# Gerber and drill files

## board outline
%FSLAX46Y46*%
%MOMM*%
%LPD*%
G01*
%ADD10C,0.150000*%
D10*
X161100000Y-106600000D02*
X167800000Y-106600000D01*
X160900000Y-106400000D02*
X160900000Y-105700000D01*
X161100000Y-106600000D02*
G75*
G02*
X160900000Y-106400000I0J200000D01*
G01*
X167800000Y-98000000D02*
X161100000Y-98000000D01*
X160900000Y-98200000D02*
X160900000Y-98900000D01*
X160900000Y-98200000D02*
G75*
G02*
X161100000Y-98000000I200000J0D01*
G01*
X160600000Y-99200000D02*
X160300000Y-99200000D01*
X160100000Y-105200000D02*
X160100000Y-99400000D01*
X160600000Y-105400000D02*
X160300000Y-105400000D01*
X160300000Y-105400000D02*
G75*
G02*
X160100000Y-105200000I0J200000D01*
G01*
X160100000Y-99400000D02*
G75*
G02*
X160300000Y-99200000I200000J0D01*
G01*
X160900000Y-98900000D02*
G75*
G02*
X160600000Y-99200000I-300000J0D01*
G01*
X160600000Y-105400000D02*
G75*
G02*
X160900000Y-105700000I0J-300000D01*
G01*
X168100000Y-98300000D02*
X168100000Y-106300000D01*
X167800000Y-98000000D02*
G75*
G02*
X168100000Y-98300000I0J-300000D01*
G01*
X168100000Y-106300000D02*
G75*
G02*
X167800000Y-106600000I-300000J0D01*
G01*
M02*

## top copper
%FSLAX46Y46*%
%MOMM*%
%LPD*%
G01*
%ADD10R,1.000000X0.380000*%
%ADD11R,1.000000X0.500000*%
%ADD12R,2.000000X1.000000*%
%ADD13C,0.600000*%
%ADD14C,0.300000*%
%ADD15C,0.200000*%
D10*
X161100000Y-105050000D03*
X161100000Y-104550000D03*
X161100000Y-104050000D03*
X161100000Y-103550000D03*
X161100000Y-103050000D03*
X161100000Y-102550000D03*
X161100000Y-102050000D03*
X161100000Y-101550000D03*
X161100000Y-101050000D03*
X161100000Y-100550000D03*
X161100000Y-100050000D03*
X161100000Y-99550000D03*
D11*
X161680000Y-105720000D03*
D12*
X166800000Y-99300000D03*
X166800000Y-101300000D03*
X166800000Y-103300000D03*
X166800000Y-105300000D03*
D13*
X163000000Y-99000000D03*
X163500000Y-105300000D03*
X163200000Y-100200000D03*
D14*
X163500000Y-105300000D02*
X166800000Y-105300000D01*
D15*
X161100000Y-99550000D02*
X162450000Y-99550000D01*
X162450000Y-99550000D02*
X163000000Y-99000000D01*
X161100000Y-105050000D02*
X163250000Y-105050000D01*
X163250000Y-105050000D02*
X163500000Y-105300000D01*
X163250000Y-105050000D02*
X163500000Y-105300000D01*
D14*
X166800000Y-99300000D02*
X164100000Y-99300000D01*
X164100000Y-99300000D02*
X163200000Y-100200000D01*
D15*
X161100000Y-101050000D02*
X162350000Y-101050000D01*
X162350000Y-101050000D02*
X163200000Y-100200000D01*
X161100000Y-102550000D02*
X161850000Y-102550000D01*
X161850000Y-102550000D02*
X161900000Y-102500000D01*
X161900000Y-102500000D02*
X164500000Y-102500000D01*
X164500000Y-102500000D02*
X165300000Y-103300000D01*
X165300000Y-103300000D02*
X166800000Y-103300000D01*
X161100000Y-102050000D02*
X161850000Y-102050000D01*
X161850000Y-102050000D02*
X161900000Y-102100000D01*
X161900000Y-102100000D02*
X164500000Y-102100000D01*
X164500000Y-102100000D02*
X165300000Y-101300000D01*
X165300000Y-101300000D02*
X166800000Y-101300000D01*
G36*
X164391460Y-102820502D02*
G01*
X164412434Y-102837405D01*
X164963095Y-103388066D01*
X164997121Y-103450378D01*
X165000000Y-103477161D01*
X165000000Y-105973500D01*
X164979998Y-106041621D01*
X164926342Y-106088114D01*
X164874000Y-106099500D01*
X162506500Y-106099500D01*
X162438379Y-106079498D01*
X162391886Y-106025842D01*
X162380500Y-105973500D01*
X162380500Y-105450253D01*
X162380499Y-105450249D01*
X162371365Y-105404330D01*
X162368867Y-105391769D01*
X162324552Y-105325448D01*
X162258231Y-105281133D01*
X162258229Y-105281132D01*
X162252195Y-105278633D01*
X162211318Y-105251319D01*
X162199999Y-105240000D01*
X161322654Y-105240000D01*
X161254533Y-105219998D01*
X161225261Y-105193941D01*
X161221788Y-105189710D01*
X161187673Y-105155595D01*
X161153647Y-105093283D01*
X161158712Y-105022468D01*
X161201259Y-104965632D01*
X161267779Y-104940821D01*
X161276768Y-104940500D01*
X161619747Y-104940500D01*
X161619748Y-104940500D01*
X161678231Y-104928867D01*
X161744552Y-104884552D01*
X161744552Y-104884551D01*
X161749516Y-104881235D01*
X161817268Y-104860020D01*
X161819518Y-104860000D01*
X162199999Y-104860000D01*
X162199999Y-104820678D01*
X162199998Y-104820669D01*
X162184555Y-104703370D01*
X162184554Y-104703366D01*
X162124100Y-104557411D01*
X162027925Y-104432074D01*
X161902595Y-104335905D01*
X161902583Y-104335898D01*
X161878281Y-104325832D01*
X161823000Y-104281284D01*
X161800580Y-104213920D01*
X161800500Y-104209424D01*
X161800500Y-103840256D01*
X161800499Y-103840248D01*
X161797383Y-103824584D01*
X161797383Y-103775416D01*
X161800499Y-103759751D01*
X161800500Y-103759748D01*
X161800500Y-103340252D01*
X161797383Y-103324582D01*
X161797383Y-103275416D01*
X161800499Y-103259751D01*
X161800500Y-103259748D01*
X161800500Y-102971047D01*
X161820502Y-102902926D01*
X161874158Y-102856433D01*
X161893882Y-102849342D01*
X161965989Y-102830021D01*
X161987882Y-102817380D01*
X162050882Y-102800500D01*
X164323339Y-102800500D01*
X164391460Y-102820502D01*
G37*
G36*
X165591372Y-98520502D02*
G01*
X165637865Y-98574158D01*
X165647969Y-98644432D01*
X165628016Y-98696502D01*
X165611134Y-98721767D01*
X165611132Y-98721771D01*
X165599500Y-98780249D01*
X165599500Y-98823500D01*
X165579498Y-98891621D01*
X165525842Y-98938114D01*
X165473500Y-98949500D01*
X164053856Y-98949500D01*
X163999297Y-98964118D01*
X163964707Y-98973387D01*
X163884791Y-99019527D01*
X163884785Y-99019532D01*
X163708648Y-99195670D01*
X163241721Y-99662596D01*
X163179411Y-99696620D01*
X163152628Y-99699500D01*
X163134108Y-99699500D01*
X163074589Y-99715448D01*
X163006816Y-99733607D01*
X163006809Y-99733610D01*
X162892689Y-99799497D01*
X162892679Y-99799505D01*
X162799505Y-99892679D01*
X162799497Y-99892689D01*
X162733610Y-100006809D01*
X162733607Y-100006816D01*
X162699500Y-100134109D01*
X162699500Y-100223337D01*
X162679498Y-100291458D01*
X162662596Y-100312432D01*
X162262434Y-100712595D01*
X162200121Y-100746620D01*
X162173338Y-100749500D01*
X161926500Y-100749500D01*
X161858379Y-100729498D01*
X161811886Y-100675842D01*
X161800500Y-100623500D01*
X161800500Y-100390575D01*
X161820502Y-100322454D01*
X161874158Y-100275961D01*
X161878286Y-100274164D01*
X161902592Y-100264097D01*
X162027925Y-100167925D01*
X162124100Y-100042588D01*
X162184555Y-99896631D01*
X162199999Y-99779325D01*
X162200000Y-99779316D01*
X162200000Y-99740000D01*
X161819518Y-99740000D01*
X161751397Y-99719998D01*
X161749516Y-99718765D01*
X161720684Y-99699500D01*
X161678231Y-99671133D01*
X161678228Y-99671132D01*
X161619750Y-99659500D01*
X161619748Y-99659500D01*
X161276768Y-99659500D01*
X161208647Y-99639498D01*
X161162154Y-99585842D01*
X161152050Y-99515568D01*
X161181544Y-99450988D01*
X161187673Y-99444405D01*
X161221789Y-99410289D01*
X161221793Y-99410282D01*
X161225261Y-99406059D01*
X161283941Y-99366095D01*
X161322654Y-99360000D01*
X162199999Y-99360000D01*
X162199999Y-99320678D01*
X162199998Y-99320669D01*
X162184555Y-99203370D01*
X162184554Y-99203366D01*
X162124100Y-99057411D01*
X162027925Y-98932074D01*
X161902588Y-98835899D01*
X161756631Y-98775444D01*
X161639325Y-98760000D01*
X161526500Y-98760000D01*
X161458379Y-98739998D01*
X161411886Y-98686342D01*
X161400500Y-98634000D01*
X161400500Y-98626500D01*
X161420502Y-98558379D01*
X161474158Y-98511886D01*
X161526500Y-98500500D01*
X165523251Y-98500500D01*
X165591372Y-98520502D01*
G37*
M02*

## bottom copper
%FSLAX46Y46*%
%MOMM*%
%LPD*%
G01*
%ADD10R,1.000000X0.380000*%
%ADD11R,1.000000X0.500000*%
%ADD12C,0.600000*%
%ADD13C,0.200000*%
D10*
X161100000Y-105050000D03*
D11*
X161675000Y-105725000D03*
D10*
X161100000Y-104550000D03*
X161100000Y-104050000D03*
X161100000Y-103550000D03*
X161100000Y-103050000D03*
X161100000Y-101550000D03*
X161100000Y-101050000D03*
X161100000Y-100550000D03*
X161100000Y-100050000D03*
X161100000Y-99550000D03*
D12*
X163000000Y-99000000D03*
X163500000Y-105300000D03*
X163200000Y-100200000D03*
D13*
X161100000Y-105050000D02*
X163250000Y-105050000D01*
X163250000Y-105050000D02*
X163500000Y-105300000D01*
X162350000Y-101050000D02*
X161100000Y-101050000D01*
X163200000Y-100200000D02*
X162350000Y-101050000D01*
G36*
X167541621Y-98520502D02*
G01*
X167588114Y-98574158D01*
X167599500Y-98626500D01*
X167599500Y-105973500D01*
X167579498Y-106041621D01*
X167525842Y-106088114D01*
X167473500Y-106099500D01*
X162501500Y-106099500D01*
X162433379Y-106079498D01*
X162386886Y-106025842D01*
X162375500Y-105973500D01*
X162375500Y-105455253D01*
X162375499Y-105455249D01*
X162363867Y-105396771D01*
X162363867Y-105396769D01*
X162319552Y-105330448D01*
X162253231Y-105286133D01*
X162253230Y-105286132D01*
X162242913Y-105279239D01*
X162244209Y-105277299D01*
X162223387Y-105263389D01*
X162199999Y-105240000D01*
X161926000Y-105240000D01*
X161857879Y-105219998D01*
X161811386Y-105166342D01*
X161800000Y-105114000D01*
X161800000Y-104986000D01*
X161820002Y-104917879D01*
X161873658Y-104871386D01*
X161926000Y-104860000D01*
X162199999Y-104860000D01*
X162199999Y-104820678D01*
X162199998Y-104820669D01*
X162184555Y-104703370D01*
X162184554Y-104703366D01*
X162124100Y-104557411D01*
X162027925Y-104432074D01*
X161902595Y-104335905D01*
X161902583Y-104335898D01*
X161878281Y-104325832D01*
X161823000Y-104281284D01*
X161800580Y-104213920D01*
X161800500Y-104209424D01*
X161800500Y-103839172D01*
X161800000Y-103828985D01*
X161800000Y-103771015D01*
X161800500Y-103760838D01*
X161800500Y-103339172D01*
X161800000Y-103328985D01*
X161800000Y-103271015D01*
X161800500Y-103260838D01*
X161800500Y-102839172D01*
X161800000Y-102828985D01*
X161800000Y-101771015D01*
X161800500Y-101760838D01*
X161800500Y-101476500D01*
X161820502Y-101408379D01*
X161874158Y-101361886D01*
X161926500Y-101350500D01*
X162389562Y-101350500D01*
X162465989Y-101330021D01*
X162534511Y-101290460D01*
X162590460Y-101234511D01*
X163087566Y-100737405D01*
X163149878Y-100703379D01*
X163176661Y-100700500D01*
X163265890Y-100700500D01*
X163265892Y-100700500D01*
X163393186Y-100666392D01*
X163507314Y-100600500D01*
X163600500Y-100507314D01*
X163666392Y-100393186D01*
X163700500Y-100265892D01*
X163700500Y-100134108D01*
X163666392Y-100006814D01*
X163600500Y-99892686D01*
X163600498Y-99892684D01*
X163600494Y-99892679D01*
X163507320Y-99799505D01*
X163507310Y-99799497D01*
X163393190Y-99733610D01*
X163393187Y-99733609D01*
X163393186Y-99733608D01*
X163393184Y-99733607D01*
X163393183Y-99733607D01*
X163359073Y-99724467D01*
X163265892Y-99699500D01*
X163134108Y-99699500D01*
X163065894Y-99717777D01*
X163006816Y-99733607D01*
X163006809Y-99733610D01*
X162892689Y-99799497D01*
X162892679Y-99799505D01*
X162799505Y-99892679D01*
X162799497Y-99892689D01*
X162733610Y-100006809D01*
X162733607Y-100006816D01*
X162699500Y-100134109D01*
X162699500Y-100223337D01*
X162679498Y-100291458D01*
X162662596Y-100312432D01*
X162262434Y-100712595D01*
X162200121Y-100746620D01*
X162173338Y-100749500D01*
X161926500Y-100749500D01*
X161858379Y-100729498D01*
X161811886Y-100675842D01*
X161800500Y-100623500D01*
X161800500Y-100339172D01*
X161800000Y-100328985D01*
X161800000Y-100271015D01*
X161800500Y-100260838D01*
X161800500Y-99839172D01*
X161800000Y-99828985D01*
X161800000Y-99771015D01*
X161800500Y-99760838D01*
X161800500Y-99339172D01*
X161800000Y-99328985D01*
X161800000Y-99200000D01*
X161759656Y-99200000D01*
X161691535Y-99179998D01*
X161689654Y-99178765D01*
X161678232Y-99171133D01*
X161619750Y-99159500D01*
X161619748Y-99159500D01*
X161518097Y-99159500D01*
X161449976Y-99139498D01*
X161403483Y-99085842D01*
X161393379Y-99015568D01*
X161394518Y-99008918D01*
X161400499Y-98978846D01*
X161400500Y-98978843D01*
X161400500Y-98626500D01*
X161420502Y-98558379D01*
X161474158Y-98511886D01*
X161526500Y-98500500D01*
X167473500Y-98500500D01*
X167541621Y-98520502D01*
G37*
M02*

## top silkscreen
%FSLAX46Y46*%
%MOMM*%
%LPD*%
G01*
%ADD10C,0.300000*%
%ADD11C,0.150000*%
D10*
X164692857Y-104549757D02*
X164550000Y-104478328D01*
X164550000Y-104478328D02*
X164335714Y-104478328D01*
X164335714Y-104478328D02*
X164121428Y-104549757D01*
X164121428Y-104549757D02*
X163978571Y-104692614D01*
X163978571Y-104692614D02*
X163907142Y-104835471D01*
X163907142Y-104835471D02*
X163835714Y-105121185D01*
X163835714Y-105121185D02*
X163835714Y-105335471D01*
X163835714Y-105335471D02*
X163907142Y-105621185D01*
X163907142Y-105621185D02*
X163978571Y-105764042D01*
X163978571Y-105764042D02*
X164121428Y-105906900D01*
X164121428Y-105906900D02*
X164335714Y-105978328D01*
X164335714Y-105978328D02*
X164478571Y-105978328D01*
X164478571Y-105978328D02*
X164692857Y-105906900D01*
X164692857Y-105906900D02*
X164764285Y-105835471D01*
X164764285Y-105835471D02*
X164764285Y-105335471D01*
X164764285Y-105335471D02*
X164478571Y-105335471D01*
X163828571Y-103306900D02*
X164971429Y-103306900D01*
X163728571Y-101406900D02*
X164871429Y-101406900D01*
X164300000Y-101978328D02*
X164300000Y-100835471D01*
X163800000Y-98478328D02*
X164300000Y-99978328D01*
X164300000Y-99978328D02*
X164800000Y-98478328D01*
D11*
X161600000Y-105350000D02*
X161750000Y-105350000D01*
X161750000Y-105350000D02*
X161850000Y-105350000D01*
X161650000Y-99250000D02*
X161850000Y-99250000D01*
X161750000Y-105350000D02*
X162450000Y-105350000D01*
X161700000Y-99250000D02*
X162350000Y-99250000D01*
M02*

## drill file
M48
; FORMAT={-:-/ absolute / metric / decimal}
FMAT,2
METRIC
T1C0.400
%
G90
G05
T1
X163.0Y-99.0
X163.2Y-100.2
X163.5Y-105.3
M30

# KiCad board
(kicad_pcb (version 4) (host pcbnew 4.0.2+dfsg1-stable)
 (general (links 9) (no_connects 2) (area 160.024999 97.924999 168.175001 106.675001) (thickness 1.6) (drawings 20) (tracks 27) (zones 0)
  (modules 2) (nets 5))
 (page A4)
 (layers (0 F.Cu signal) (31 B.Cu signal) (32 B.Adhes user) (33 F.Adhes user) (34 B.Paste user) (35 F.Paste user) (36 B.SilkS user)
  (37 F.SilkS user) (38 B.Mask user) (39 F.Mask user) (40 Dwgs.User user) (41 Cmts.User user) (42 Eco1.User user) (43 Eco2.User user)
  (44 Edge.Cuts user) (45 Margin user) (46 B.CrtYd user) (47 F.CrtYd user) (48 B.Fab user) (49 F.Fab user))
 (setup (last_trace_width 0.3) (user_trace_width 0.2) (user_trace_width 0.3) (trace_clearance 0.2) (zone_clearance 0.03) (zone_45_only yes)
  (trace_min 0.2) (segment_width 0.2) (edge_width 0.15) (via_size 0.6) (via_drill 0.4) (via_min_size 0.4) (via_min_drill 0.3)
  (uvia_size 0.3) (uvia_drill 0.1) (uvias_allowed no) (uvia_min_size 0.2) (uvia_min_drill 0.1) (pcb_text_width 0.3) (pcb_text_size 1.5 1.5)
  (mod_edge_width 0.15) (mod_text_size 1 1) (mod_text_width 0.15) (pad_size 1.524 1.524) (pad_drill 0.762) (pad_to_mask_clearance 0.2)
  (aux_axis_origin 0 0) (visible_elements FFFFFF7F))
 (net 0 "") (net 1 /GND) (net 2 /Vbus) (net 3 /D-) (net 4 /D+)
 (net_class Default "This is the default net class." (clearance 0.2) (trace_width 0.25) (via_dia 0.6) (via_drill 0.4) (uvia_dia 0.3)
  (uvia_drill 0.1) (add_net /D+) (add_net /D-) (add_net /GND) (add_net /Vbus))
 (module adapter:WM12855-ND (layer F.Cu) (at 163.6 102.3 90)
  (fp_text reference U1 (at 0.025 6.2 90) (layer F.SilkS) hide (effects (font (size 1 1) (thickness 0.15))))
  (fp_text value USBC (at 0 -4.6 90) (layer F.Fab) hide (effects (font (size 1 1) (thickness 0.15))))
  (fp_line (start -3.05 -2) (end -3.05 -1.85) (layer F.SilkS) (width 0.15))
  (fp_line (start -3.05 -1.85) (end -3.05 -1.75) (layer F.SilkS) (width 0.15))
  (fp_line (start 3.05 -1.95) (end 3.05 -1.75) (layer F.SilkS) (width 0.15))
  (fp_line (start -3.05 -1.85) (end -3.05 -1.15) (layer F.SilkS) (width 0.15))
  (fp_line (start 3.05 -1.9) (end 3.05 -1.25) (layer F.SilkS) (width 0.15))
  (pad B1 smd rect (at -2.75 -2.5 90) (size 0.38 1) (layers B.Cu B.Paste B.Mask) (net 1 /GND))
  (pad X smd rect (at -3.425 -1.925 90) (size 0.5 1) (layers B.Cu B.Paste B.Mask))
  (pad A12 smd rect (at -2.75 -2.5 90) (size 0.38 1) (layers F.Cu F.Paste F.Mask) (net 1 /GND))
  (pad A11 smd rect (at -2.25 -2.5 90) (size 0.38 1) (layers F.Cu F.Paste F.Mask))
  (pad A10 smd rect (at -1.75 -2.5 90) (size 0.38 1) (layers F.Cu F.Paste F.Mask))
  (pad A9 smd rect (at -1.25 -2.5 90) (size 0.38 1) (layers F.Cu F.Paste F.Mask) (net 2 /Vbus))
  (pad A8 smd rect (at -0.75 -2.5 90) (size 0.38 1) (layers F.Cu F.Paste F.Mask))
  (pad A7 smd rect (at -0.25 -2.5 90) (size 0.38 1) (layers F.Cu F.Paste F.Mask) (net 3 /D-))
  (pad A6 smd rect (at 0.25 -2.5 90) (size 0.38 1) (layers F.Cu F.Paste F.Mask) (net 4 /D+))
  (pad A5 smd rect (at 0.75 -2.5 90) (size 0.38 1) (layers F.Cu F.Paste F.Mask))
  (pad A4 smd rect (at 1.25 -2.5 90) (size 0.38 1) (layers F.Cu F.Paste F.Mask) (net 2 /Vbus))
  (pad A3 smd rect (at 1.75 -2.5 90) (size 0.38 1) (layers F.Cu F.Paste F.Mask))
  (pad A2 smd rect (at 2.25 -2.5 90) (size 0.38 1) (layers F.Cu F.Paste F.Mask))
  (pad A1 smd rect (at 2.75 -2.5 90) (size 0.38 1) (layers F.Cu F.Paste F.Mask) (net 1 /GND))
  (pad X smd rect (at -3.42 -1.92 90) (size 0.5 1) (layers F.Cu F.Paste F.Mask))
  (pad B2 smd rect (at -2.25 -2.5 90) (size 0.38 1) (layers B.Cu B.Paste B.Mask))
  (pad B3 smd rect (at -1.75 -2.5 90) (size 0.38 1) (layers B.Cu B.Paste B.Mask))
  (pad B4 smd rect (at -1.25 -2.5 90) (size 0.38 1) (layers B.Cu B.Paste B.Mask) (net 2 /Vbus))
  (pad B5 smd rect (at -0.75 -2.5 90) (size 0.38 1) (layers B.Cu B.Paste B.Mask))
  (pad B8 smd rect (at 0.75 -2.5 90) (size 0.38 1) (layers B.Cu B.Paste B.Mask))
  (pad B9 smd rect (at 1.25 -2.5 90) (size 0.38 1) (layers B.Cu B.Paste B.Mask) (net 2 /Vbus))
  (pad B10 smd rect (at 1.75 -2.5 90) (size 0.38 1) (layers B.Cu B.Paste B.Mask))
  (pad B11 smd rect (at 2.25 -2.5 90) (size 0.38 1) (layers B.Cu B.Paste B.Mask))
  (pad B12 smd rect (at 2.75 -2.5 90) (size 0.38 1) (layers B.Cu B.Paste B.Mask)))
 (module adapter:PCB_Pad (layer F.Cu) (at 163.8 102.3 90)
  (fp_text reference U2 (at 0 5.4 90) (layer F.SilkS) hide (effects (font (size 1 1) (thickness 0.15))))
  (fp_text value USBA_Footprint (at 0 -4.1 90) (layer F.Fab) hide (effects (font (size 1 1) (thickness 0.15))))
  (pad Vbus smd rect (at 3 3 90) (size 1 2) (layers F.Cu F.Paste F.Mask) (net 2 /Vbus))
  (pad D+ smd rect (at 1 3 90) (size 1 2) (layers F.Cu F.Paste F.Mask) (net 4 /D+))
  (pad D- smd rect (at -1 3 90) (size 1 2) (layers F.Cu F.Paste F.Mask) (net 3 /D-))
  (pad GND smd rect (at -3 3 90) (size 1 2) (layers F.Cu F.Paste F.Mask) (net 1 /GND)))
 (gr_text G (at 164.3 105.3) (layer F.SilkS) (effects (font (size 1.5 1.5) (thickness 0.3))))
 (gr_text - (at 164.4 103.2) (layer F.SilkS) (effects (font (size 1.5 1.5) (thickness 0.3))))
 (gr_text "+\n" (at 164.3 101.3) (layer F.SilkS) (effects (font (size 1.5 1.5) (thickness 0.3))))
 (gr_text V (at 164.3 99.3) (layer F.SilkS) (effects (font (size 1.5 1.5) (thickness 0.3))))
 (gr_line (start 161.1 106.6) (end 167.8 106.6) (angle 90) (layer Edge.Cuts) (width 0.15))
 (gr_line (start 160.9 106.4) (end 160.9 105.7) (angle 90) (layer Edge.Cuts) (width 0.15))
 (gr_arc (start 161.1 106.4) (end 161.1 106.6) (angle 90) (layer Edge.Cuts) (width 0.15))
 (gr_line (start 167.8 98) (end 161.1 98) (angle 90) (layer Edge.Cuts) (width 0.15))
 (gr_line (start 160.9 98.2) (end 160.9 98.9) (angle 90) (layer Edge.Cuts) (width 0.15))
 (gr_arc (start 161.1 98.2) (end 160.9 98.2) (angle 90) (layer Edge.Cuts) (width 0.15))
 (gr_line (start 160.6 99.2) (end 160.3 99.2) (angle 90) (layer Edge.Cuts) (width 0.15))
 (gr_line (start 160.1 105.2) (end 160.1 99.4) (angle 90) (layer Edge.Cuts) (width 0.15))
 (gr_line (start 160.6 105.4) (end 160.3 105.4) (angle 90) (layer Edge.Cuts) (width 0.15))
 (gr_arc (start 160.3 105.2) (end 160.3 105.4) (angle 90) (layer Edge.Cuts) (width 0.15))
 (gr_arc (start 160.3 99.4) (end 160.1 99.4) (angle 90) (layer Edge.Cuts) (width 0.15))
 (gr_arc (start 160.6 98.9) (end 160.9 98.9) (angle 90) (layer Edge.Cuts) (width 0.15))
 (gr_arc (start 160.6 105.7) (end 160.6 105.4) (angle 90) (layer Edge.Cuts) (width 0.15))
 (gr_line (start 168.1 98.3) (end 168.1 106.3) (angle 90) (layer Edge.Cuts) (width 0.15))
 (gr_arc (start 167.8 98.3) (end 167.8 98) (angle 90) (layer Edge.Cuts) (width 0.15))
 (gr_arc (start 167.8 106.3) (end 168.1 106.3) (angle 90) (layer Edge.Cuts) (width 0.15))
 (segment (start 163.5 105.3) (end 166.8 105.3) (width 0.3) (layer F.Cu) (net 1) (status 800000))
 (segment (start 161.1 99.55) (end 162.45 99.55) (width 0.2) (layer F.Cu) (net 1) (status 400000))
 (via (at 163 99) (size 0.6) (drill 0.4) (layers F.Cu B.Cu) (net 1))
 (segment (start 162.45 99.55) (end 163 99) (width 0.2) (layer F.Cu) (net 1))
 (segment (start 161.1 105.05) (end 163.25 105.05) (width 0.2) (layer F.Cu) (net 1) (status 400000))
 (segment (start 163.25 105.05) (end 163.5 105.3) (width 0.2) (layer F.Cu) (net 1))
 (segment (start 161.1 105.05) (end 163.25 105.05) (width 0.2) (layer B.Cu) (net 1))
 (segment (start 163.25 105.05) (end 163.5 105.3) (width 0.2) (layer F.Cu) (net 1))
 (via (at 163.5 105.3) (size 0.6) (drill 0.4) (layers F.Cu B.Cu) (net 1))
 (segment (start 163.25 105.05) (end 163.5 105.3) (width 0.2) (layer B.Cu) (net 1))
 (segment (start 166.8 99.3) (end 164.1 99.3) (width 0.3) (layer F.Cu) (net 2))
 (segment (start 164.1 99.3) (end 163.2 100.2) (width 0.3) (layer F.Cu) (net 2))
 (segment (start 161.1 101.05) (end 162.35 101.05) (width 0.2) (layer F.Cu) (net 2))
 (segment (start 162.35 101.05) (end 163.2 100.2) (width 0.2) (layer F.Cu) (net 2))
 (segment (start 162.35 101.05) (end 161.1 101.05) (width 0.2) (layer B.Cu) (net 2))
 (segment (start 163.2 100.2) (end 162.35 101.05) (width 0.2) (layer B.Cu) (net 2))
 (via (at 163.2 100.2) (size 0.6) (drill 0.4) (layers F.Cu B.Cu) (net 2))
 (segment (start 161.1 102.55) (end 161.85 102.55) (width 0.2) (layer F.Cu) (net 3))
 (segment (start 161.85 102.55) (end 161.9 102.5) (width 0.2) (layer F.Cu) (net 3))
 (segment (start 161.9 102.5) (end 164.5 102.5) (width 0.2) (layer F.Cu) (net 3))
 (segment (start 164.5 102.5) (end 165.3 103.3) (width 0.2) (layer F.Cu) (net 3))
 (segment (start 165.3 103.3) (end 166.8 103.3) (width 0.2) (layer F.Cu) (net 3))
 (segment (start 161.1 102.05) (end 161.85 102.05) (width 0.2) (layer F.Cu) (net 4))
 (segment (start 161.85 102.05) (end 161.9 102.1) (width 0.2) (layer F.Cu) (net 4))
 (segment (start 161.9 102.1) (end 164.5 102.1) (width 0.2) (layer F.Cu) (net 4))
 (segment (start 164.5 102.1) (end 165.3 101.3) (width 0.2) (layer F.Cu) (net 4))
 (segment (start 165.3 101.3) (end 166.8 101.3) (width 0.2) (layer F.Cu) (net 4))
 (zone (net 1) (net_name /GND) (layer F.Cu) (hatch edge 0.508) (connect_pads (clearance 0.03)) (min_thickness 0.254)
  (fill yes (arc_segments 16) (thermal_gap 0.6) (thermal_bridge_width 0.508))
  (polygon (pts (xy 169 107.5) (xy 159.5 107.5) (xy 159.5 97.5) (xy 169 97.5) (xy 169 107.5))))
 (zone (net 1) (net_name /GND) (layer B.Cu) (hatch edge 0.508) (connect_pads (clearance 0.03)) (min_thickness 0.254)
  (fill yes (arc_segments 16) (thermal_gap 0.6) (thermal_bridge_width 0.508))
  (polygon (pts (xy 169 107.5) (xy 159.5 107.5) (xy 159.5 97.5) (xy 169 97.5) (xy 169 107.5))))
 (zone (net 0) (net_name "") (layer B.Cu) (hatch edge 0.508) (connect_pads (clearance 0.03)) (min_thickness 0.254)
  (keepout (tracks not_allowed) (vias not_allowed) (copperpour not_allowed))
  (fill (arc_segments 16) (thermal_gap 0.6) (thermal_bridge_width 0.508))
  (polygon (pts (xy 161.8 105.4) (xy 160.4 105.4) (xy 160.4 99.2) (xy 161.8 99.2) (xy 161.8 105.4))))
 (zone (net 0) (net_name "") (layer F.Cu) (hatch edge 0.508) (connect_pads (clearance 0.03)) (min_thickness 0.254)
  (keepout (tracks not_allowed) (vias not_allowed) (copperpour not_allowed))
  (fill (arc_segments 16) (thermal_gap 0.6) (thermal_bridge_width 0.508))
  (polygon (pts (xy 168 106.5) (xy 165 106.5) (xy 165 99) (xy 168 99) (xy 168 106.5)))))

